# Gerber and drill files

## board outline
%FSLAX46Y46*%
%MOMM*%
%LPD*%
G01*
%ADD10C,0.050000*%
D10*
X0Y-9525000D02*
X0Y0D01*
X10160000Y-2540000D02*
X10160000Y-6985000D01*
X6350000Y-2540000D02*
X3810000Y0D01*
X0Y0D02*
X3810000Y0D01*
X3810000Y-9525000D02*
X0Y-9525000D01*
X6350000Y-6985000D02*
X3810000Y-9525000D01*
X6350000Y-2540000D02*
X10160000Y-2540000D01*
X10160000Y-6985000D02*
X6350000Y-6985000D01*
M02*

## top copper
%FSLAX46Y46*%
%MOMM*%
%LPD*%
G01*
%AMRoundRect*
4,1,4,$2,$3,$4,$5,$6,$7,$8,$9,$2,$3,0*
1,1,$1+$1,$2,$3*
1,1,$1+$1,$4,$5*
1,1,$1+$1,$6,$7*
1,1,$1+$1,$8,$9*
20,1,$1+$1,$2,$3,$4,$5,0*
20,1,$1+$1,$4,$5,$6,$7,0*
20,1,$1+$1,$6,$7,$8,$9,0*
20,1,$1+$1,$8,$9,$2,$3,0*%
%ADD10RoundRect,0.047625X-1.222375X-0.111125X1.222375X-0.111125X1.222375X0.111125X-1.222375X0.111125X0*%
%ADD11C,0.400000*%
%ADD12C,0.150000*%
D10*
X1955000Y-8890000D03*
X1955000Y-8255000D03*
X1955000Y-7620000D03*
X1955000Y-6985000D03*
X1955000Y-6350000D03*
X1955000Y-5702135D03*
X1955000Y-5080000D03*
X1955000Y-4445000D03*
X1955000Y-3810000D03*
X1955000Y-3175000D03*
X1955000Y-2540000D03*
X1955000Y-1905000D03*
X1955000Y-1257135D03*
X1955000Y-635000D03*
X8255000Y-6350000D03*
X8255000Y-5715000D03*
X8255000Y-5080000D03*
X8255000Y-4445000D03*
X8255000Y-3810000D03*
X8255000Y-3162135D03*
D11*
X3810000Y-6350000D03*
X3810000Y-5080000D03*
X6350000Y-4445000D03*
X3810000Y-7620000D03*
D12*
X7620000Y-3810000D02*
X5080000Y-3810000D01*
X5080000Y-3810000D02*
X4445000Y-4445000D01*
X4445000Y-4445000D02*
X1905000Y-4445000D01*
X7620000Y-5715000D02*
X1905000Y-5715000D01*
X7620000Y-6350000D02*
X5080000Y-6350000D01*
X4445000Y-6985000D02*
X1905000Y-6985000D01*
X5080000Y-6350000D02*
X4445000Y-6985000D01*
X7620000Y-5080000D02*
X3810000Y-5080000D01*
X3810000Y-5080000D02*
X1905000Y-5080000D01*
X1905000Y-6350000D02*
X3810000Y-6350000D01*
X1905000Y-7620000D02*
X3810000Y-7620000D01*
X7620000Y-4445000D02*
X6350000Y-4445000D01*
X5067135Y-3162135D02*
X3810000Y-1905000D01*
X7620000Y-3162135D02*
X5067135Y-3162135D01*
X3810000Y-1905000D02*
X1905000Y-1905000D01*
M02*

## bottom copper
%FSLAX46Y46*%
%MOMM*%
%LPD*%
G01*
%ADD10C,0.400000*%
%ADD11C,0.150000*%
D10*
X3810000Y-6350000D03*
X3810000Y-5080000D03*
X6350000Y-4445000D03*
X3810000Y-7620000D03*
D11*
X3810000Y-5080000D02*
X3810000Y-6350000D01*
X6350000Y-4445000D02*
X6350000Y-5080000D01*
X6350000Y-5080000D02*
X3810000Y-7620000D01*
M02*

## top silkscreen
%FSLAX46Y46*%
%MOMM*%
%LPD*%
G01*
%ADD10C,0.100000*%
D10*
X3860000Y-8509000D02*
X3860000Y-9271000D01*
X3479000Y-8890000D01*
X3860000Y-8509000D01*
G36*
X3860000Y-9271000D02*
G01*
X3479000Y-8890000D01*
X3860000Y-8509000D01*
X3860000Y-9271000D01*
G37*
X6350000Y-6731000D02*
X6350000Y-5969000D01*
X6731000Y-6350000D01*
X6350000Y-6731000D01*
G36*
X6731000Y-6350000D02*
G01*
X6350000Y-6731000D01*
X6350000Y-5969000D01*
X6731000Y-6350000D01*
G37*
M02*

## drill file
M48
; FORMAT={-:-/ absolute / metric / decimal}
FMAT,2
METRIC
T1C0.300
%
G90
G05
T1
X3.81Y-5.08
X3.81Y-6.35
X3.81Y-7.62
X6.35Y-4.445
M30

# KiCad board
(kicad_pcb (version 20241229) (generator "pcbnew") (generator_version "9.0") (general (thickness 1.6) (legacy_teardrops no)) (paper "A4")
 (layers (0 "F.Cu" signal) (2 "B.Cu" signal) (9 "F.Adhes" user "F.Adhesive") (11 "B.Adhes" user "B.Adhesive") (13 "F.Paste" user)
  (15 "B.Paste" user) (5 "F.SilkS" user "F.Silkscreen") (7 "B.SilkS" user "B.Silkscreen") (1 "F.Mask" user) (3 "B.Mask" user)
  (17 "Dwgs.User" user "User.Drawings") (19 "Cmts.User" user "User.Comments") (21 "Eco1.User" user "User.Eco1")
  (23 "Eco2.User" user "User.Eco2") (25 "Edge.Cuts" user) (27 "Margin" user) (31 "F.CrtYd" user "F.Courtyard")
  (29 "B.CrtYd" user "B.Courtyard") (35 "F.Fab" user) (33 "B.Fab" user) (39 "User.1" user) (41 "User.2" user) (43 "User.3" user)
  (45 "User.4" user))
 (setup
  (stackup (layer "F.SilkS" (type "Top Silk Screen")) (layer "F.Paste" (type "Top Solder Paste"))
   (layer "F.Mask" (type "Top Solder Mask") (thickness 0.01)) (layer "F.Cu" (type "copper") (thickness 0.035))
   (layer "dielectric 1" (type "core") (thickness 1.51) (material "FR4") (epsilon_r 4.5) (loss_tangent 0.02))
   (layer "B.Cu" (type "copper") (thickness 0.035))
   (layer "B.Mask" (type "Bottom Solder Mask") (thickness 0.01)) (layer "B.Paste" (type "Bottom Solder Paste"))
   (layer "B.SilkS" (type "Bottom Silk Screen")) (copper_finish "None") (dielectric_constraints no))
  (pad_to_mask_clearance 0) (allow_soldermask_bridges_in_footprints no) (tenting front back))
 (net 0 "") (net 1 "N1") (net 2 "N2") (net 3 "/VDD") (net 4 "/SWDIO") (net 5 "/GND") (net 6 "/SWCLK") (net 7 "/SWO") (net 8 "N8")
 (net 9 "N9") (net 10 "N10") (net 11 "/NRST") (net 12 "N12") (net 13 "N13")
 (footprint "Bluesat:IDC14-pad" (layer "F.Cu") (at 1.955 0.635)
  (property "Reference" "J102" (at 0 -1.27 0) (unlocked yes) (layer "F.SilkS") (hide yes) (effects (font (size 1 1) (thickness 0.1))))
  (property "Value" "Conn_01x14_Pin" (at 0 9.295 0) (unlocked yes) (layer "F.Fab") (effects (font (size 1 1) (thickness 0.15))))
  (fp_poly (pts (xy 1.905 7.874) (xy 1.905 8.636) (xy 1.524 8.255)) (stroke (width 0.1) (type solid)) (fill yes) (layer "F.SilkS"))
  (pad "1" smd roundrect (at 0 8.255) (size 2.54 0.3175) (layers "F.Cu" "F.Mask" "F.Paste") (roundrect_rratio 0.15) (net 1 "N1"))
  (pad "2" smd roundrect (at 0 7.62) (size 2.54 0.3175) (layers "F.Cu" "F.Mask" "F.Paste") (roundrect_rratio 0.15) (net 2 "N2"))
  (pad "3" smd roundrect (at 0 6.985) (size 2.54 0.3175) (layers "F.Cu" "F.Mask" "F.Paste") (roundrect_rratio 0.15) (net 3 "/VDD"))
  (pad "4" smd roundrect (at 0 6.35) (size 2.54 0.3175) (layers "F.Cu" "F.Mask" "F.Paste") (roundrect_rratio 0.15) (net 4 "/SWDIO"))
  (pad "5" smd roundrect (at 0 5.715) (size 2.54 0.3175) (layers "F.Cu" "F.Mask" "F.Paste") (roundrect_rratio 0.15) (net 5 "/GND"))
  (pad "6" smd roundrect (at 0 5.067135) (size 2.54 0.3175) (layers "F.Cu" "F.Mask" "F.Paste") (roundrect_rratio 0.15) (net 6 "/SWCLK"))
  (pad "7" smd roundrect (at 0 4.445) (size 2.54 0.3175) (layers "F.Cu" "F.Mask" "F.Paste") (roundrect_rratio 0.15) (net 5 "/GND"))
  (pad "8" smd roundrect (at 0 3.81) (size 2.54 0.3175) (layers "F.Cu" "F.Mask" "F.Paste") (roundrect_rratio 0.15) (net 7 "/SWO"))
  (pad "9" smd roundrect (at 0 3.175) (size 2.54 0.3175) (layers "F.Cu" "F.Mask" "F.Paste") (roundrect_rratio 0.15) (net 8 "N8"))
  (pad "10" smd roundrect (at 0 2.54) (size 2.54 0.3175) (layers "F.Cu" "F.Mask" "F.Paste") (roundrect_rratio 0.15) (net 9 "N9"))
  (pad "11" smd roundrect (at 0 1.905) (size 2.54 0.3175) (layers "F.Cu" "F.Mask" "F.Paste") (roundrect_rratio 0.15) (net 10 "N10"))
  (pad "12" smd roundrect (at 0 1.27) (size 2.54 0.3175) (layers "F.Cu" "F.Mask" "F.Paste") (roundrect_rratio 0.15) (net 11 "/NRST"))
  (pad "13" smd roundrect (at 0 0.622135) (size 2.54 0.3175) (layers "F.Cu" "F.Mask" "F.Paste") (roundrect_rratio 0.15) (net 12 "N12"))
  (pad "14" smd roundrect (at 0 0) (size 2.54 0.3175) (layers "F.Cu" "F.Mask" "F.Paste") (roundrect_rratio 0.15) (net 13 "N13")))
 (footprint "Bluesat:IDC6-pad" (layer "F.Cu") (at 8.255 3.175)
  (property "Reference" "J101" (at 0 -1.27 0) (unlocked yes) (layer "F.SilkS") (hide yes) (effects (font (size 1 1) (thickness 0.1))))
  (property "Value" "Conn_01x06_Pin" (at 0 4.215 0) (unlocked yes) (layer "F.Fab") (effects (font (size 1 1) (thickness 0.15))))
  (fp_poly (pts (xy -1.905 3.556) (xy -1.905 2.794) (xy -1.524 3.175)) (stroke (width 0.1) (type solid)) (fill yes) (layer "F.SilkS"))
  (pad "1" smd roundrect (at 0 3.175) (size 2.54 0.3175) (layers "F.Cu" "F.Mask" "F.Paste") (roundrect_rratio 0.15) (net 4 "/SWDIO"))
  (pad "2" smd roundrect (at 0 2.54) (size 2.54 0.3175) (layers "F.Cu" "F.Mask" "F.Paste") (roundrect_rratio 0.15) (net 6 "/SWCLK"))
  (pad "3" smd roundrect (at 0 1.905) (size 2.54 0.3175) (layers "F.Cu" "F.Mask" "F.Paste") (roundrect_rratio 0.15) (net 5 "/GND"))
  (pad "4" smd roundrect (at 0 1.27) (size 2.54 0.3175) (layers "F.Cu" "F.Mask" "F.Paste") (roundrect_rratio 0.15) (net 3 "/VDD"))
  (pad "5" smd roundrect (at 0 0.635) (size 2.54 0.3175) (layers "F.Cu" "F.Mask" "F.Paste") (roundrect_rratio 0.15) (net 7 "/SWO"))
  (pad "6" smd roundrect (at 0 -0.012865) (size 2.54 0.3175) (layers "F.Cu" "F.Mask" "F.Paste") (roundrect_rratio 0.15) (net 11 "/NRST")))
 (gr_line (start 0 9.525) (end 0 0) (stroke (width 0.05) (type default)) (layer "Edge.Cuts"))
 (gr_line (start 10.16 2.54) (end 10.16 6.985) (stroke (width 0.05) (type default)) (layer "Edge.Cuts"))
 (gr_line (start 6.35 2.54) (end 3.81 0) (stroke (width 0.05) (type default)) (layer "Edge.Cuts"))
 (gr_line (start 0 0) (end 3.81 0) (stroke (width 0.05) (type default)) (layer "Edge.Cuts"))
 (gr_line (start 3.81 9.525) (end 0 9.525) (stroke (width 0.05) (type default)) (layer "Edge.Cuts"))
 (gr_line (start 6.35 6.985) (end 3.81 9.525) (stroke (width 0.05) (type default)) (layer "Edge.Cuts"))
 (gr_line (start 6.35 2.54) (end 10.16 2.54) (stroke (width 0.05) (type default)) (layer "Edge.Cuts"))
 (gr_line (start 10.16 6.985) (end 6.35 6.985) (stroke (width 0.05) (type default)) (layer "Edge.Cuts"))
 (segment (start 7.62 3.81) (end 5.08 3.81) (width 0.15) (layer "F.Cu") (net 7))
 (segment (start 5.08 3.81) (end 4.445 4.445) (width 0.15) (layer "F.Cu") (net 7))
 (segment (start 4.445 4.445) (end 1.905 4.445) (width 0.15) (layer "F.Cu") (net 7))
 (segment (start 7.62 5.715) (end 1.905 5.715) (width 0.15) (layer "F.Cu") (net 6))
 (segment (start 7.62 6.35) (end 5.08 6.35) (width 0.15) (layer "F.Cu") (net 4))
 (segment (start 4.445 6.985) (end 1.905 6.985) (width 0.15) (layer "F.Cu") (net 4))
 (segment (start 5.08 6.35) (end 4.445 6.985) (width 0.15) (layer "F.Cu") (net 4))
 (segment (start 7.62 5.08) (end 3.81 5.08) (width 0.15) (layer "F.Cu") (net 5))
 (segment (start 3.81 5.08) (end 1.905 5.08) (width 0.15) (layer "F.Cu") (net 5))
 (segment (start 1.905 6.35) (end 3.81 6.35) (width 0.15) (layer "F.Cu") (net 5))
 (via (at 3.81 6.35) (size 0.4) (drill 0.3) (layers "F.Cu" "B.Cu") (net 5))
 (via (at 3.81 5.08) (size 0.4) (drill 0.3) (layers "F.Cu" "B.Cu") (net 5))
 (segment (start 3.81 5.08) (end 3.81 6.35) (width 0.15) (layer "B.Cu") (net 5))
 (segment (start 1.905 7.62) (end 3.81 7.62) (width 0.15) (layer "F.Cu") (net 3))
 (segment (start 7.62 4.445) (end 6.35 4.445) (width 0.15) (layer "F.Cu") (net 3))
 (via (at 6.35 4.445) (size 0.4) (drill 0.3) (layers "F.Cu" "B.Cu") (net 3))
 (via (at 3.81 7.62) (size 0.4) (drill 0.3) (layers "F.Cu" "B.Cu") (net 3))
 (segment (start 6.35 4.445) (end 6.35 5.08) (width 0.15) (layer "B.Cu") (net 3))
 (segment (start 6.35 5.08) (end 3.81 7.62) (width 0.15) (layer "B.Cu") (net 3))
 (segment (start 5.067135 3.162135) (end 3.81 1.905) (width 0.15) (layer "F.Cu") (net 11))
 (segment (start 7.62 3.162135) (end 5.067135 3.162135) (width 0.15) (layer "F.Cu") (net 11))
 (segment (start 3.81 1.905) (end 1.905 1.905) (width 0.15) (layer "F.Cu") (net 11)))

